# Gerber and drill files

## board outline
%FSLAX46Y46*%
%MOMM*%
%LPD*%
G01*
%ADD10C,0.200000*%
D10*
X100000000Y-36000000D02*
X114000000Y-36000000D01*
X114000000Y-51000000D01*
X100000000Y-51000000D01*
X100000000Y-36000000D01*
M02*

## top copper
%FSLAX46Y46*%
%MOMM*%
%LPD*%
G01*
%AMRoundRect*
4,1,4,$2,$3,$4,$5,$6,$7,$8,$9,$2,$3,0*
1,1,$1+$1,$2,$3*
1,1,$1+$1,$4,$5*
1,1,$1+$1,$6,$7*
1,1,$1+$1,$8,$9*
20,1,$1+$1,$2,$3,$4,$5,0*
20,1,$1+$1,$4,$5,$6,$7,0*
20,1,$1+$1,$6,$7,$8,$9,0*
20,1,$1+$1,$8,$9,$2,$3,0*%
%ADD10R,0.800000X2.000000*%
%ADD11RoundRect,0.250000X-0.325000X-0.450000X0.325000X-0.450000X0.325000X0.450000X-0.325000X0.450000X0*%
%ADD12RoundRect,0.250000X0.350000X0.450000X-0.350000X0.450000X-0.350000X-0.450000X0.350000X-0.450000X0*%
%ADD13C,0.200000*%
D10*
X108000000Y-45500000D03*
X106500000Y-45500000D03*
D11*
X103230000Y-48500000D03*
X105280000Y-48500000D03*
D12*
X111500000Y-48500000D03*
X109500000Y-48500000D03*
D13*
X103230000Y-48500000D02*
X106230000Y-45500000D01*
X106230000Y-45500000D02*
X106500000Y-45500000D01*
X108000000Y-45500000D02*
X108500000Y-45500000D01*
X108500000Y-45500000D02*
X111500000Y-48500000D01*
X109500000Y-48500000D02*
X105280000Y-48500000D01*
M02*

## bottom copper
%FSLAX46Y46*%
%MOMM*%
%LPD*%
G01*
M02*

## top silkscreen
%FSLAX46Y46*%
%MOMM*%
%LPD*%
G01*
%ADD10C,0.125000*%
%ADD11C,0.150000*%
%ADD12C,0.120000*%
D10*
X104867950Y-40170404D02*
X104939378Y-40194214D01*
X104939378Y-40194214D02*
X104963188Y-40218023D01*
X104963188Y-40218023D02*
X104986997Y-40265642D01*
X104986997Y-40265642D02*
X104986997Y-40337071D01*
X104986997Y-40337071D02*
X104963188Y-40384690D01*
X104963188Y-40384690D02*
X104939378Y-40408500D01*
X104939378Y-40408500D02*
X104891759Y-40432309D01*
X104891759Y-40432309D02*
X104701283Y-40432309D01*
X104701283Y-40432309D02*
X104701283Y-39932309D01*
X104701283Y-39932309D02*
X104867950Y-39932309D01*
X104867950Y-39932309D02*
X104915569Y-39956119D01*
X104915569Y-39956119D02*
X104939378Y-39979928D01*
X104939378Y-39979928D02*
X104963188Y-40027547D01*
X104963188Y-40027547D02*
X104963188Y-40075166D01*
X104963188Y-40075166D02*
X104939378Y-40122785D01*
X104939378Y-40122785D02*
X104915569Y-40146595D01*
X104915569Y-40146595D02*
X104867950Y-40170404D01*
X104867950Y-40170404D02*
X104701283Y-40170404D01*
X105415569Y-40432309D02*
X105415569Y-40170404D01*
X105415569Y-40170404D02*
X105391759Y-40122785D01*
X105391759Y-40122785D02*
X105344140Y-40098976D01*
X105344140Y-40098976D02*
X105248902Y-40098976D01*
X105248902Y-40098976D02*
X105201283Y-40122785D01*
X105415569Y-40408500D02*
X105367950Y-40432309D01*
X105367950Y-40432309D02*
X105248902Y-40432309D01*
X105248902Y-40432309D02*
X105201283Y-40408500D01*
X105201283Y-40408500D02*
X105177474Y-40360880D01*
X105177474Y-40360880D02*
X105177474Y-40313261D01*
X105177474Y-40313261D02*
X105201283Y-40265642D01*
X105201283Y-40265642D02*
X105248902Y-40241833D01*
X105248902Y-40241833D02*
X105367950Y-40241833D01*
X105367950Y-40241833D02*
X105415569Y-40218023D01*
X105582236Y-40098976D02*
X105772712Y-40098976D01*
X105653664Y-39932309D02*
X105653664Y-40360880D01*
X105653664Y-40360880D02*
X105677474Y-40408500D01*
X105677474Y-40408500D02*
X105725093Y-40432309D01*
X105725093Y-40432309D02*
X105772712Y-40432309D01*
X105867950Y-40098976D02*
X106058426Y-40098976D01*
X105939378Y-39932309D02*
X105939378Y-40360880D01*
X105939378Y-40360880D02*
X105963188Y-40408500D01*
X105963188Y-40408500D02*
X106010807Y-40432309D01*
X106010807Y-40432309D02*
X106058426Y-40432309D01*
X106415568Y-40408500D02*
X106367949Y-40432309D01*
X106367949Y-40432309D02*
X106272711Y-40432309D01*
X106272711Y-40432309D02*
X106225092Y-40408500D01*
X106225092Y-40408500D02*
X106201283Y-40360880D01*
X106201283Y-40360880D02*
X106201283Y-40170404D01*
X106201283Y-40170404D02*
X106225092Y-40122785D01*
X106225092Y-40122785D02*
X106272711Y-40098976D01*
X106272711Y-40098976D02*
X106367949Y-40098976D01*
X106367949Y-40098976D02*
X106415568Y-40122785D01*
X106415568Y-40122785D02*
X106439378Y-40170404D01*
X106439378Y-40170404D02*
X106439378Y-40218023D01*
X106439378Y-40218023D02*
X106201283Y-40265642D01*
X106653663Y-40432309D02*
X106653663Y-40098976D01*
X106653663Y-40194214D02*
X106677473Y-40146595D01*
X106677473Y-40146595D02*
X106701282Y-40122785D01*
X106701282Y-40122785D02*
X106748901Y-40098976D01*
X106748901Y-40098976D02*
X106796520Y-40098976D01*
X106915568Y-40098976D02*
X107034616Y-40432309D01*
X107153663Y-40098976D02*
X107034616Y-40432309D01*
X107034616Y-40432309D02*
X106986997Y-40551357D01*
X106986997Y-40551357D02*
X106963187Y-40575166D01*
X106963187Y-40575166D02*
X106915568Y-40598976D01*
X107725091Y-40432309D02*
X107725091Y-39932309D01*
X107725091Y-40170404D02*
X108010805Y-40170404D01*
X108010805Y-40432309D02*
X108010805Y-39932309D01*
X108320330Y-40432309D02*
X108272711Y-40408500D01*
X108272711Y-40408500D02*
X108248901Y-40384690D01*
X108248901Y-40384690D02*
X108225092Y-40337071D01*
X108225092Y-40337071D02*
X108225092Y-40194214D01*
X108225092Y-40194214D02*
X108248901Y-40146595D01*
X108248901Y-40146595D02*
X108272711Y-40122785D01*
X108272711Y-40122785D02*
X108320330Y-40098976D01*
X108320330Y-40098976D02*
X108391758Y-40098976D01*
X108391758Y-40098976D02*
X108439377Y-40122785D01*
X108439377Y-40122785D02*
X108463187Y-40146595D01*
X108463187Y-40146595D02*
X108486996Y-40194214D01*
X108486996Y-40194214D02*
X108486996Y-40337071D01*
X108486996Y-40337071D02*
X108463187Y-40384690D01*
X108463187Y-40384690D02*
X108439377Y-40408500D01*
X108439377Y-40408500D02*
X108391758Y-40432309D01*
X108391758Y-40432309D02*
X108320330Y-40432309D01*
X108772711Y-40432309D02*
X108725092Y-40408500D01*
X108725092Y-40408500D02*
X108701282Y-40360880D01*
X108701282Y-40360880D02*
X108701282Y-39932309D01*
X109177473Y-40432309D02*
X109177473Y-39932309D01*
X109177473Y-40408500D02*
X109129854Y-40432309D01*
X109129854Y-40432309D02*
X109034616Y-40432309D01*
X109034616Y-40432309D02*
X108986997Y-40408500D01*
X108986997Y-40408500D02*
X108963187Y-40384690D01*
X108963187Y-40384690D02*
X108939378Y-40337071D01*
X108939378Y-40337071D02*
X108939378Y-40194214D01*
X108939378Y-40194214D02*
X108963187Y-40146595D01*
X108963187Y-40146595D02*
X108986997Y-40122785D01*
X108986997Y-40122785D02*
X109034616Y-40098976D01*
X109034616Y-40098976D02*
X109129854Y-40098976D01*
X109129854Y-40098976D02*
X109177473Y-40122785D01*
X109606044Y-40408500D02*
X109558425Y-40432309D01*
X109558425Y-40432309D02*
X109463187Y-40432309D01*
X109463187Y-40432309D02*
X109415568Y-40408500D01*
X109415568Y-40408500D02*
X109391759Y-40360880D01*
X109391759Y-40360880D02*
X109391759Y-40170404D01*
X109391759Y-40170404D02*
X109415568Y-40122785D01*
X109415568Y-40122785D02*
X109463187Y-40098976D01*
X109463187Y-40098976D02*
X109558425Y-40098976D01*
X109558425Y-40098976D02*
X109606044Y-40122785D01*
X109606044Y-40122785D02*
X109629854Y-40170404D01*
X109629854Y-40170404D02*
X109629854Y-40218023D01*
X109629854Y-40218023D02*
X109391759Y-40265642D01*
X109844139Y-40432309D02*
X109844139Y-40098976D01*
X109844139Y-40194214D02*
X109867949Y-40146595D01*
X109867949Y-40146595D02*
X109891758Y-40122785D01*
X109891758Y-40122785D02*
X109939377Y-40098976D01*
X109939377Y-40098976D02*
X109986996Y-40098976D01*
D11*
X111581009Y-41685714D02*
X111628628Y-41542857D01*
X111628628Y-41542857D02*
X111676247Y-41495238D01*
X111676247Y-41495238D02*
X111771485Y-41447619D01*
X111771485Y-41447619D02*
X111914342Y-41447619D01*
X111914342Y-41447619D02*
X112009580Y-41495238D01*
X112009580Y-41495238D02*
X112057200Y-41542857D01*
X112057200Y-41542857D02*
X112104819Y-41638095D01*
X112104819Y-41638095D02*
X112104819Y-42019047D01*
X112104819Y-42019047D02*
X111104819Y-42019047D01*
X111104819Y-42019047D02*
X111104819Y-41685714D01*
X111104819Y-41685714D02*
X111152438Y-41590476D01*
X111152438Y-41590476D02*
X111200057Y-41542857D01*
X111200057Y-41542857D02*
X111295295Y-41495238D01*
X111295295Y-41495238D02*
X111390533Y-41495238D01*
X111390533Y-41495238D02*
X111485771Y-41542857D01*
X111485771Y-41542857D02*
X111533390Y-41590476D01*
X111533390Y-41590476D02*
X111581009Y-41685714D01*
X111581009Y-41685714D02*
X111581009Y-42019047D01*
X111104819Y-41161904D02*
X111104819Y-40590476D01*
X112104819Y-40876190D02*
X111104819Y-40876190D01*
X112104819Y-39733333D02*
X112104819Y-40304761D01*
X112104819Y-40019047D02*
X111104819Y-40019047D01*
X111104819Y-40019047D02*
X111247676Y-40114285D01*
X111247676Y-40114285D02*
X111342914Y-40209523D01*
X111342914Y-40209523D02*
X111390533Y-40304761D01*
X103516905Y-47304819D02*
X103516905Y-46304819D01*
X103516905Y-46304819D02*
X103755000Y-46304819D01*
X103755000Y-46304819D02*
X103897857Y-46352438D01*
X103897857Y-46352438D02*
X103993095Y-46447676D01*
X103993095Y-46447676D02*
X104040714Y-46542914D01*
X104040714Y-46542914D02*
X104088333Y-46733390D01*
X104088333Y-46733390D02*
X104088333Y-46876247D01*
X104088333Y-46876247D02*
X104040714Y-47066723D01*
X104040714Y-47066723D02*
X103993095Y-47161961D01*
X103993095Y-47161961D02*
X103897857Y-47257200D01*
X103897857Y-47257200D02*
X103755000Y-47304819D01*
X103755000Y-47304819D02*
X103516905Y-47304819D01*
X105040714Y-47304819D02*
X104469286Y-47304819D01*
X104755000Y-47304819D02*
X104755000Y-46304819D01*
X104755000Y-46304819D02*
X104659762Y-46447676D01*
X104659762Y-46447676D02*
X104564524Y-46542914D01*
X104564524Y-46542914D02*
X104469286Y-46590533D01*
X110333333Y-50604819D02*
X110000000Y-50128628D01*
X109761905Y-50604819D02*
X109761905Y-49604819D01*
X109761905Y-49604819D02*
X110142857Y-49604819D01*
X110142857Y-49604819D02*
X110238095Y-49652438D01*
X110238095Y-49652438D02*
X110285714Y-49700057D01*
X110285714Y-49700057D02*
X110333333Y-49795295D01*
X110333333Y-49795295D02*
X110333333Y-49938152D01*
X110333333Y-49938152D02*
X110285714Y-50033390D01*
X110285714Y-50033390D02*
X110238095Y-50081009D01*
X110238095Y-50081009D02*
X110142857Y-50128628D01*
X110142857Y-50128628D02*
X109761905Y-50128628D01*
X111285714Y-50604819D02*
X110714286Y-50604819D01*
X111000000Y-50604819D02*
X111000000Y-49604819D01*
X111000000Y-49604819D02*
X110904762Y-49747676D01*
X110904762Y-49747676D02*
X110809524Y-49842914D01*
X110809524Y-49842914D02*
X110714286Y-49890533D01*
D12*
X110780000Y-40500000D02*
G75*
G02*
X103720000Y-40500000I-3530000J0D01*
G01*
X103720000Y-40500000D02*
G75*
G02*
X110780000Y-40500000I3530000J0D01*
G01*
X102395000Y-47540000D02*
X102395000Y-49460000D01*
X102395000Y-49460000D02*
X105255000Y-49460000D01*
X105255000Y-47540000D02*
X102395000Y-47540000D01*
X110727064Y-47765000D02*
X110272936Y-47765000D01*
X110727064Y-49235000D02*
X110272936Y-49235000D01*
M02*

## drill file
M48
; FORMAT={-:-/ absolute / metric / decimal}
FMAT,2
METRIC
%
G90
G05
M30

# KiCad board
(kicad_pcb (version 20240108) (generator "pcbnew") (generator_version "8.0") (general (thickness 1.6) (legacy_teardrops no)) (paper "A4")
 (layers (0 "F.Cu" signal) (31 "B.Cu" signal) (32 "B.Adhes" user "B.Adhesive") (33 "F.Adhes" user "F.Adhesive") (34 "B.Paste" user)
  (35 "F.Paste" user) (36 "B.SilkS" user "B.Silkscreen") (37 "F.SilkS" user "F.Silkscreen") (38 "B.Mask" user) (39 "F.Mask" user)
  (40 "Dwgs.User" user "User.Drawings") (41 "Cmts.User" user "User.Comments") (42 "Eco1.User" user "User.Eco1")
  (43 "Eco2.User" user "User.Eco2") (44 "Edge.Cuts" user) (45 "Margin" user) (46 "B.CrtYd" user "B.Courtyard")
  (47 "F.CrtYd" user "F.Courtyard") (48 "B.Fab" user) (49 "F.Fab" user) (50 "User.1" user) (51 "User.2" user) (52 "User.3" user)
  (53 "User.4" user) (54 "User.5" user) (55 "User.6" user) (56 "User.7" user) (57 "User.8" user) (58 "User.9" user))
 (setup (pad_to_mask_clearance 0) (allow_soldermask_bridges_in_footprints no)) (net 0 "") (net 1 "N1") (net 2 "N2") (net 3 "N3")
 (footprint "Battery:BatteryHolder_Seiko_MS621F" (layer "F.Cu") (at 107.25 45.5 -90)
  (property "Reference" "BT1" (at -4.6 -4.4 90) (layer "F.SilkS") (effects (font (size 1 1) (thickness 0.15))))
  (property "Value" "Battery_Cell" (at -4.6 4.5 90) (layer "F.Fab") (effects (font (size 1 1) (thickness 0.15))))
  (fp_circle (center -5 0) (end -1.47 0) (stroke (width 0.12) (type solid)) (fill none) (layer "F.SilkS"))
  (pad "1" smd rect (at 0 -0.75 270) (size 2 0.8) (layers "F.Cu" "F.Paste" "F.Mask") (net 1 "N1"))
  (pad "2" smd rect (at 0 0.75 270) (size 2 0.8) (layers "F.Cu" "F.Paste" "F.Mask") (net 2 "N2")))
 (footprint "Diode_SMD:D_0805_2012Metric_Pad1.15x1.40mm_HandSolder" (layer "F.Cu") (at 104.255 48.5)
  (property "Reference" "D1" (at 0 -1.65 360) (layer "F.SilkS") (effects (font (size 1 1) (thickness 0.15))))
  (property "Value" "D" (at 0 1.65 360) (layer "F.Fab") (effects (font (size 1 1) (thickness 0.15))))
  (fp_line (start -1.86 -0.96) (end -1.86 0.96) (stroke (width 0.12) (type solid)) (layer "F.SilkS"))
  (fp_line (start -1.86 0.96) (end 1 0.96) (stroke (width 0.12) (type solid)) (layer "F.SilkS"))
  (fp_line (start 1 -0.96) (end -1.86 -0.96) (stroke (width 0.12) (type solid)) (layer "F.SilkS"))
  (pad "1" smd roundrect (at -1.025 0) (size 1.15 1.4) (layers "F.Cu" "F.Paste" "F.Mask") (roundrect_rratio 0.217391) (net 2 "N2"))
  (pad "2" smd roundrect (at 1.025 0) (size 1.15 1.4) (layers "F.Cu" "F.Paste" "F.Mask") (roundrect_rratio 0.217391) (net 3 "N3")))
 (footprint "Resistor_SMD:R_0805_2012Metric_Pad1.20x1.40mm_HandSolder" (layer "F.Cu") (at 110.5 48.5 180)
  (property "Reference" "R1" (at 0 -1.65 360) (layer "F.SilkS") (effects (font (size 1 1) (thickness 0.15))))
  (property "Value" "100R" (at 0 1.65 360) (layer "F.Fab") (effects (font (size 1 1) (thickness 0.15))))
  (fp_line (start -0.227064 0.735) (end 0.227064 0.735) (stroke (width 0.12) (type solid)) (layer "F.SilkS"))
  (fp_line (start -0.227064 -0.735) (end 0.227064 -0.735) (stroke (width 0.12) (type solid)) (layer "F.SilkS"))
  (pad "1" smd roundrect (at -1 0 180) (size 1.2 1.4) (layers "F.Cu" "F.Paste" "F.Mask") (roundrect_rratio 0.208333) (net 1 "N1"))
  (pad "2" smd roundrect (at 1 0 180) (size 1.2 1.4) (layers "F.Cu" "F.Paste" "F.Mask") (roundrect_rratio 0.208333) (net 3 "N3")))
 (gr_rect (start 100 36) (end 114 51) (stroke (width 0.2) (type default)) (fill none) (layer "Edge.Cuts"))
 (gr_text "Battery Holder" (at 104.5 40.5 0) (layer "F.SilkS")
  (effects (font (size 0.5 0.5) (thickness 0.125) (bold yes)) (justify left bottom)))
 (segment (start 103.23 48.5) (end 106.23 45.5) (width 0.2) (layer "F.Cu") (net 2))
 (segment (start 106.23 45.5) (end 106.5 45.5) (width 0.2) (layer "F.Cu") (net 2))
 (segment (start 108 45.5) (end 108.5 45.5) (width 0.2) (layer "F.Cu") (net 1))
 (segment (start 108.5 45.5) (end 111.5 48.5) (width 0.2) (layer "F.Cu") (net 1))
 (segment (start 109.5 48.5) (end 105.28 48.5) (width 0.2) (layer "F.Cu") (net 3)))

